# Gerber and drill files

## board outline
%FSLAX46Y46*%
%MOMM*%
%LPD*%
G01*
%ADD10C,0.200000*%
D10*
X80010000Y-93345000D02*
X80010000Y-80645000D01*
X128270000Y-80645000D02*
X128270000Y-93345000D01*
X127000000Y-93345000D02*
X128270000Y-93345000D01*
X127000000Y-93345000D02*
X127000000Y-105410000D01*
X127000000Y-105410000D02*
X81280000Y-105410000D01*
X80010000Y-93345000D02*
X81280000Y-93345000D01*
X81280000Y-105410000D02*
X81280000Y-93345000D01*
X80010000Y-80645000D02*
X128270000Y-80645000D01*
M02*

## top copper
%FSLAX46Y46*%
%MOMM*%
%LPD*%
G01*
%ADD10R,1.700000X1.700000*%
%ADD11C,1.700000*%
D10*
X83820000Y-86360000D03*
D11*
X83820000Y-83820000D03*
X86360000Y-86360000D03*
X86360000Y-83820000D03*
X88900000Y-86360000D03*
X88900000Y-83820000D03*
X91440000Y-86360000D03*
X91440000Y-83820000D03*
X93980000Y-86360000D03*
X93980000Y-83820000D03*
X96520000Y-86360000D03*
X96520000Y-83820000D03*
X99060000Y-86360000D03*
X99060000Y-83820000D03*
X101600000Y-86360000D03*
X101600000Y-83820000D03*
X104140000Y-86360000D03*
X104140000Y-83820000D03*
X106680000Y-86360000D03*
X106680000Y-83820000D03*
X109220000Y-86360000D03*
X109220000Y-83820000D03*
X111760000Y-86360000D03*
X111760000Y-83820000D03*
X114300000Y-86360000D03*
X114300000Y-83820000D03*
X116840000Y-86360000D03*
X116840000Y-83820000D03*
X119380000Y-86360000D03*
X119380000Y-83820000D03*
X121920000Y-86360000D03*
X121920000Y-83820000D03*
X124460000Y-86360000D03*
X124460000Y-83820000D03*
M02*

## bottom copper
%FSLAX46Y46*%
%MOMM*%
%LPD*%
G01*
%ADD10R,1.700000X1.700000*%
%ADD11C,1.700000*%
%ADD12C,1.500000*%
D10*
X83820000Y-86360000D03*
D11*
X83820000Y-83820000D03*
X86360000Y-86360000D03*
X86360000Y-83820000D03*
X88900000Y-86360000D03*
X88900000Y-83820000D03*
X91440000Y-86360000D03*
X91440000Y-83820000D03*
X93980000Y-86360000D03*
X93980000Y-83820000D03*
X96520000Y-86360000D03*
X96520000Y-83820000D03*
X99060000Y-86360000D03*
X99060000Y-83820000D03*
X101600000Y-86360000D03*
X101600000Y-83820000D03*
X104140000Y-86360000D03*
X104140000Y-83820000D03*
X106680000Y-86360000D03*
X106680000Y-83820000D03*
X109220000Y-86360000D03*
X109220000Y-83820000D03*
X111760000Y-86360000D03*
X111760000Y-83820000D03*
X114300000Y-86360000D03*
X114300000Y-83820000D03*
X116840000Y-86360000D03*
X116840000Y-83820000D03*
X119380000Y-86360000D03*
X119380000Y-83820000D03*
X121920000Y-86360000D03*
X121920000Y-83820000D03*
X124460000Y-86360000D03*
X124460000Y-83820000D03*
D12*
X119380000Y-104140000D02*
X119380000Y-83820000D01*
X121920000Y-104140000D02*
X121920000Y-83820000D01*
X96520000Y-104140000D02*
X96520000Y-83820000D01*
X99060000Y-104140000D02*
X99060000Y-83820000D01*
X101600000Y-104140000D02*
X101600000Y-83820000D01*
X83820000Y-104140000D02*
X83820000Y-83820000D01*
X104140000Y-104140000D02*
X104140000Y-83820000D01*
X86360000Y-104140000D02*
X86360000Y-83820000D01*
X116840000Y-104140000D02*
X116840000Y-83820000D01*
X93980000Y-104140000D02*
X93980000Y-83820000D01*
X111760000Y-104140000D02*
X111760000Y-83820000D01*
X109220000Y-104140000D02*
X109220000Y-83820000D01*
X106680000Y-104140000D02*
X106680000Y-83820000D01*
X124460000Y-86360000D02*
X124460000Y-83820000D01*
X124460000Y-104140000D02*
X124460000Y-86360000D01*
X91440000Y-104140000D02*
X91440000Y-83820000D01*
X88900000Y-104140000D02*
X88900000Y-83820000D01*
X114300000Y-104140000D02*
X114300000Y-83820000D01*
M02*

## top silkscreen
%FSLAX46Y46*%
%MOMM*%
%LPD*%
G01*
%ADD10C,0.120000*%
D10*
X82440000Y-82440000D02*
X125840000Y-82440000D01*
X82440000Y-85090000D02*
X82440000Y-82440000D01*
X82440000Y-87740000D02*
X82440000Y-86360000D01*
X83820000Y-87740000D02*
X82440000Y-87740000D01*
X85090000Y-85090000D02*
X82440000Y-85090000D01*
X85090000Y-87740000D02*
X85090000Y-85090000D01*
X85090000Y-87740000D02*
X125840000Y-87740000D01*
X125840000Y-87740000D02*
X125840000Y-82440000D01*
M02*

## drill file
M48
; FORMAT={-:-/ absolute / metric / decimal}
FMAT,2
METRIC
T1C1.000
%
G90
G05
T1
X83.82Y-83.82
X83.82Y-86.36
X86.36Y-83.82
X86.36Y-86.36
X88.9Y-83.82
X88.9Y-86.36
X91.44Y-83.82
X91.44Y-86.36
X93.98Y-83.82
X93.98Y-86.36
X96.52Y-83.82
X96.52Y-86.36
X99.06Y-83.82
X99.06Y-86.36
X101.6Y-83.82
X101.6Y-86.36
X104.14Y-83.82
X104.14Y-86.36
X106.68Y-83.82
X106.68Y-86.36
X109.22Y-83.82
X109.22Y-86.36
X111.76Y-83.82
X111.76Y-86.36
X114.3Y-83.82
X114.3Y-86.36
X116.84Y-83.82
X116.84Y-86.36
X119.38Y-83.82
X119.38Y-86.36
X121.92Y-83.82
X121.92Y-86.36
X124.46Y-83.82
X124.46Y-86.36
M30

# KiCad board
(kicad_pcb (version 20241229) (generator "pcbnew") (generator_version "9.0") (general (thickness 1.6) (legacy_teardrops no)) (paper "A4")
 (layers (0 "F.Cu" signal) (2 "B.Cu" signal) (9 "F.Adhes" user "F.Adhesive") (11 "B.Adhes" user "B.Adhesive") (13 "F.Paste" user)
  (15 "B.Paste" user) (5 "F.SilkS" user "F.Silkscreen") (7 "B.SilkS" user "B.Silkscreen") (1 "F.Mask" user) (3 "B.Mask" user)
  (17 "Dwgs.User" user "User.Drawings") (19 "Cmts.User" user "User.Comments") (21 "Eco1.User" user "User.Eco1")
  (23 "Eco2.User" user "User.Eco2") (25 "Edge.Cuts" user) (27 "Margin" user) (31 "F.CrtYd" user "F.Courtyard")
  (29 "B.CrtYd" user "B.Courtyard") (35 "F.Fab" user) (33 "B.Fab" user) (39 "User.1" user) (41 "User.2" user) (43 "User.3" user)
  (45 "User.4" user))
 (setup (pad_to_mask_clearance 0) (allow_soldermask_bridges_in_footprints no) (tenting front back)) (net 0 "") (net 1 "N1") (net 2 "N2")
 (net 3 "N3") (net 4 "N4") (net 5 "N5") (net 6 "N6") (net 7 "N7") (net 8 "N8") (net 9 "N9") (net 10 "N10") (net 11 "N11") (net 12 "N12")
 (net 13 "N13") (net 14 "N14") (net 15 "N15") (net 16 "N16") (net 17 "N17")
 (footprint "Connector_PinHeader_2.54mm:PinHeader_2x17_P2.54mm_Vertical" (layer "F.Cu") (at 83.82 86.36 90)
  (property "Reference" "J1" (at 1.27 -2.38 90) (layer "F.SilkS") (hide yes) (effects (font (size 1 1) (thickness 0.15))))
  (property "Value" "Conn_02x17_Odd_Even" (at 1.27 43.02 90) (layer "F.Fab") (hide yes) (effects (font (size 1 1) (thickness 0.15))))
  (fp_line (start 3.92 -1.38) (end 3.92 42.02) (stroke (width 0.12) (type solid)) (layer "F.SilkS"))
  (fp_line (start 1.27 -1.38) (end 3.92 -1.38) (stroke (width 0.12) (type solid)) (layer "F.SilkS"))
  (fp_line (start -1.38 -1.38) (end 0 -1.38) (stroke (width 0.12) (type solid)) (layer "F.SilkS"))
  (fp_line (start -1.38 0) (end -1.38 -1.38) (stroke (width 0.12) (type solid)) (layer "F.SilkS"))
  (fp_line (start 1.27 1.27) (end 1.27 -1.38) (stroke (width 0.12) (type solid)) (layer "F.SilkS"))
  (fp_line (start -1.38 1.27) (end 1.27 1.27) (stroke (width 0.12) (type solid)) (layer "F.SilkS"))
  (fp_line (start -1.38 1.27) (end -1.38 42.02) (stroke (width 0.12) (type solid)) (layer "F.SilkS"))
  (fp_line (start -1.38 42.02) (end 3.92 42.02) (stroke (width 0.12) (type solid)) (layer "F.SilkS"))
  (pad "1" thru_hole rect (at 0 0 90) (size 1.7 1.7) (drill 1) (layers "*.Cu" "*.Mask") (remove_unused_layers no) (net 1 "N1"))
  (pad "2" thru_hole circle (at 2.54 0 90) (size 1.7 1.7) (drill 1) (layers "*.Cu" "*.Mask") (remove_unused_layers no) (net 1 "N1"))
  (pad "3" thru_hole circle (at 0 2.54 90) (size 1.7 1.7) (drill 1) (layers "*.Cu" "*.Mask") (remove_unused_layers no) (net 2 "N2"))
  (pad "4" thru_hole circle (at 2.54 2.54 90) (size 1.7 1.7) (drill 1) (layers "*.Cu" "*.Mask") (remove_unused_layers no) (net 2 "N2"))
  (pad "5" thru_hole circle (at 0 5.08 90) (size 1.7 1.7) (drill 1) (layers "*.Cu" "*.Mask") (remove_unused_layers no) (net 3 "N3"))
  (pad "6" thru_hole circle (at 2.54 5.08 90) (size 1.7 1.7) (drill 1) (layers "*.Cu" "*.Mask") (remove_unused_layers no) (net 3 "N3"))
  (pad "7" thru_hole circle (at 0 7.62 90) (size 1.7 1.7) (drill 1) (layers "*.Cu" "*.Mask") (remove_unused_layers no) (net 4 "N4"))
  (pad "8" thru_hole circle (at 2.54 7.62 90) (size 1.7 1.7) (drill 1) (layers "*.Cu" "*.Mask") (remove_unused_layers no) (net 4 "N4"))
  (pad "9" thru_hole circle (at 0 10.16 90) (size 1.7 1.7) (drill 1) (layers "*.Cu" "*.Mask") (remove_unused_layers no) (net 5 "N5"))
  (pad "10" thru_hole circle (at 2.54 10.16 90) (size 1.7 1.7) (drill 1) (layers "*.Cu" "*.Mask") (remove_unused_layers no) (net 5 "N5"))
  (pad "11" thru_hole circle (at 0 12.7 90) (size 1.7 1.7) (drill 1) (layers "*.Cu" "*.Mask") (remove_unused_layers no) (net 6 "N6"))
  (pad "12" thru_hole circle (at 2.54 12.7 90) (size 1.7 1.7) (drill 1) (layers "*.Cu" "*.Mask") (remove_unused_layers no) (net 6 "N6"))
  (pad "13" thru_hole circle (at 0 15.24 90) (size 1.7 1.7) (drill 1) (layers "*.Cu" "*.Mask") (remove_unused_layers no) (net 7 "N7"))
  (pad "14" thru_hole circle (at 2.54 15.24 90) (size 1.7 1.7) (drill 1) (layers "*.Cu" "*.Mask") (remove_unused_layers no) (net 7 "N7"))
  (pad "15" thru_hole circle (at 0 17.78 90) (size 1.7 1.7) (drill 1) (layers "*.Cu" "*.Mask") (remove_unused_layers no) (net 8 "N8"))
  (pad "16" thru_hole circle (at 2.54 17.78 90) (size 1.7 1.7) (drill 1) (layers "*.Cu" "*.Mask") (remove_unused_layers no) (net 8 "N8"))
  (pad "17" thru_hole circle (at 0 20.32 90) (size 1.7 1.7) (drill 1) (layers "*.Cu" "*.Mask") (remove_unused_layers no) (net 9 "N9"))
  (pad "18" thru_hole circle (at 2.54 20.32 90) (size 1.7 1.7) (drill 1) (layers "*.Cu" "*.Mask") (remove_unused_layers no) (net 9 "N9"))
  (pad "19" thru_hole circle (at 0 22.86 90) (size 1.7 1.7) (drill 1) (layers "*.Cu" "*.Mask") (remove_unused_layers no) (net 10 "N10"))
  (pad "20" thru_hole circle (at 2.54 22.86 90) (size 1.7 1.7) (drill 1) (layers "*.Cu" "*.Mask") (remove_unused_layers no) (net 10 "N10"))
  (pad "21" thru_hole circle (at 0 25.4 90) (size 1.7 1.7) (drill 1) (layers "*.Cu" "*.Mask") (remove_unused_layers no) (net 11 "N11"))
  (pad "22" thru_hole circle (at 2.54 25.4 90) (size 1.7 1.7) (drill 1) (layers "*.Cu" "*.Mask") (remove_unused_layers no) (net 11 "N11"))
  (pad "23" thru_hole circle (at 0 27.94 90) (size 1.7 1.7) (drill 1) (layers "*.Cu" "*.Mask") (remove_unused_layers no) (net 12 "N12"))
  (pad "24" thru_hole circle (at 2.54 27.94 90) (size 1.7 1.7) (drill 1) (layers "*.Cu" "*.Mask") (remove_unused_layers no) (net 12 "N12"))
  (pad "25" thru_hole circle (at 0 30.48 90) (size 1.7 1.7) (drill 1) (layers "*.Cu" "*.Mask") (remove_unused_layers no) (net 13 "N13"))
  (pad "26" thru_hole circle (at 2.54 30.48 90) (size 1.7 1.7) (drill 1) (layers "*.Cu" "*.Mask") (remove_unused_layers no) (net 13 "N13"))
  (pad "27" thru_hole circle (at 0 33.02 90) (size 1.7 1.7) (drill 1) (layers "*.Cu" "*.Mask") (remove_unused_layers no) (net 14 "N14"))
  (pad "28" thru_hole circle (at 2.54 33.02 90) (size 1.7 1.7) (drill 1) (layers "*.Cu" "*.Mask") (remove_unused_layers no) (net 14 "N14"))
  (pad "29" thru_hole circle (at 0 35.56 90) (size 1.7 1.7) (drill 1) (layers "*.Cu" "*.Mask") (remove_unused_layers no) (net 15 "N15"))
  (pad "30" thru_hole circle (at 2.54 35.56 90) (size 1.7 1.7) (drill 1) (layers "*.Cu" "*.Mask") (remove_unused_layers no) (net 15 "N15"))
  (pad "31" thru_hole circle (at 0 38.1 90) (size 1.7 1.7) (drill 1) (layers "*.Cu" "*.Mask") (remove_unused_layers no) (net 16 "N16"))
  (pad "32" thru_hole circle (at 2.54 38.1 90) (size 1.7 1.7) (drill 1) (layers "*.Cu" "*.Mask") (remove_unused_layers no) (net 16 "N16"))
  (pad "33" thru_hole circle (at 0 40.64 90) (size 1.7 1.7) (drill 1) (layers "*.Cu" "*.Mask") (remove_unused_layers no) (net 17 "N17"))
  (pad "34" thru_hole circle (at 2.54 40.64 90) (size 1.7 1.7) (drill 1) (layers "*.Cu" "*.Mask") (remove_unused_layers no) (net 17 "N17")))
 (gr_line (start 80.01 93.345) (end 80.01 80.645) (stroke (width 0.2) (type solid)) (layer "Edge.Cuts"))
 (gr_line (start 128.27 80.645) (end 128.27 93.345) (stroke (width 0.2) (type solid)) (layer "Edge.Cuts"))
 (gr_line (start 127 93.345) (end 128.27 93.345) (stroke (width 0.2) (type solid)) (layer "Edge.Cuts"))
 (gr_line (start 127 93.345) (end 127 105.41) (stroke (width 0.2) (type solid)) (layer "Edge.Cuts"))
 (gr_line (start 127 105.41) (end 81.28 105.41) (stroke (width 0.2) (type solid)) (layer "Edge.Cuts"))
 (gr_line (start 80.01 93.345) (end 81.28 93.345) (stroke (width 0.2) (type solid)) (layer "Edge.Cuts"))
 (gr_line (start 81.28 105.41) (end 81.28 93.345) (stroke (width 0.2) (type solid)) (layer "Edge.Cuts"))
 (gr_line (start 80.01 80.645) (end 128.27 80.645) (stroke (width 0.2) (type solid)) (layer "Edge.Cuts"))
 (segment (start 119.38 104.14) (end 119.38 83.82) (width 1.5) (layer "B.Cu") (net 15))
 (segment (start 121.92 104.14) (end 121.92 83.82) (width 1.5) (layer "B.Cu") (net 16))
 (segment (start 96.52 104.14) (end 96.52 83.82) (width 1.5) (layer "B.Cu") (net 6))
 (segment (start 99.06 104.14) (end 99.06 83.82) (width 1.5) (layer "B.Cu") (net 7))
 (segment (start 101.6 104.14) (end 101.6 83.82) (width 1.5) (layer "B.Cu") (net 8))
 (segment (start 83.82 104.14) (end 83.82 83.82) (width 1.5) (layer "B.Cu") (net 1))
 (segment (start 104.14 104.14) (end 104.14 83.82) (width 1.5) (layer "B.Cu") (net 9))
 (segment (start 86.36 104.14) (end 86.36 83.82) (width 1.5) (layer "B.Cu") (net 2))
 (segment (start 116.84 104.14) (end 116.84 83.82) (width 1.5) (layer "B.Cu") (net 14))
 (segment (start 93.98 104.14) (end 93.98 83.82) (width 1.5) (layer "B.Cu") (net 5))
 (segment (start 111.76 104.14) (end 111.76 83.82) (width 1.5) (layer "B.Cu") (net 12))
 (segment (start 109.22 104.14) (end 109.22 83.82) (width 1.5) (layer "B.Cu") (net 11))
 (segment (start 106.68 104.14) (end 106.68 83.82) (width 1.5) (layer "B.Cu") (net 10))
 (segment (start 124.46 86.36) (end 124.46 83.82) (width 1.5) (layer "B.Cu") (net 17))
 (segment (start 124.46 104.14) (end 124.46 86.36) (width 1.5) (layer "B.Cu") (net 17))
 (segment (start 91.44 104.14) (end 91.44 83.82) (width 1.5) (layer "B.Cu") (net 4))
 (segment (start 88.9 104.14) (end 88.9 83.82) (width 1.5) (layer "B.Cu") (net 3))
 (segment (start 114.3 104.14) (end 114.3 83.82) (width 1.5) (layer "B.Cu") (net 13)))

